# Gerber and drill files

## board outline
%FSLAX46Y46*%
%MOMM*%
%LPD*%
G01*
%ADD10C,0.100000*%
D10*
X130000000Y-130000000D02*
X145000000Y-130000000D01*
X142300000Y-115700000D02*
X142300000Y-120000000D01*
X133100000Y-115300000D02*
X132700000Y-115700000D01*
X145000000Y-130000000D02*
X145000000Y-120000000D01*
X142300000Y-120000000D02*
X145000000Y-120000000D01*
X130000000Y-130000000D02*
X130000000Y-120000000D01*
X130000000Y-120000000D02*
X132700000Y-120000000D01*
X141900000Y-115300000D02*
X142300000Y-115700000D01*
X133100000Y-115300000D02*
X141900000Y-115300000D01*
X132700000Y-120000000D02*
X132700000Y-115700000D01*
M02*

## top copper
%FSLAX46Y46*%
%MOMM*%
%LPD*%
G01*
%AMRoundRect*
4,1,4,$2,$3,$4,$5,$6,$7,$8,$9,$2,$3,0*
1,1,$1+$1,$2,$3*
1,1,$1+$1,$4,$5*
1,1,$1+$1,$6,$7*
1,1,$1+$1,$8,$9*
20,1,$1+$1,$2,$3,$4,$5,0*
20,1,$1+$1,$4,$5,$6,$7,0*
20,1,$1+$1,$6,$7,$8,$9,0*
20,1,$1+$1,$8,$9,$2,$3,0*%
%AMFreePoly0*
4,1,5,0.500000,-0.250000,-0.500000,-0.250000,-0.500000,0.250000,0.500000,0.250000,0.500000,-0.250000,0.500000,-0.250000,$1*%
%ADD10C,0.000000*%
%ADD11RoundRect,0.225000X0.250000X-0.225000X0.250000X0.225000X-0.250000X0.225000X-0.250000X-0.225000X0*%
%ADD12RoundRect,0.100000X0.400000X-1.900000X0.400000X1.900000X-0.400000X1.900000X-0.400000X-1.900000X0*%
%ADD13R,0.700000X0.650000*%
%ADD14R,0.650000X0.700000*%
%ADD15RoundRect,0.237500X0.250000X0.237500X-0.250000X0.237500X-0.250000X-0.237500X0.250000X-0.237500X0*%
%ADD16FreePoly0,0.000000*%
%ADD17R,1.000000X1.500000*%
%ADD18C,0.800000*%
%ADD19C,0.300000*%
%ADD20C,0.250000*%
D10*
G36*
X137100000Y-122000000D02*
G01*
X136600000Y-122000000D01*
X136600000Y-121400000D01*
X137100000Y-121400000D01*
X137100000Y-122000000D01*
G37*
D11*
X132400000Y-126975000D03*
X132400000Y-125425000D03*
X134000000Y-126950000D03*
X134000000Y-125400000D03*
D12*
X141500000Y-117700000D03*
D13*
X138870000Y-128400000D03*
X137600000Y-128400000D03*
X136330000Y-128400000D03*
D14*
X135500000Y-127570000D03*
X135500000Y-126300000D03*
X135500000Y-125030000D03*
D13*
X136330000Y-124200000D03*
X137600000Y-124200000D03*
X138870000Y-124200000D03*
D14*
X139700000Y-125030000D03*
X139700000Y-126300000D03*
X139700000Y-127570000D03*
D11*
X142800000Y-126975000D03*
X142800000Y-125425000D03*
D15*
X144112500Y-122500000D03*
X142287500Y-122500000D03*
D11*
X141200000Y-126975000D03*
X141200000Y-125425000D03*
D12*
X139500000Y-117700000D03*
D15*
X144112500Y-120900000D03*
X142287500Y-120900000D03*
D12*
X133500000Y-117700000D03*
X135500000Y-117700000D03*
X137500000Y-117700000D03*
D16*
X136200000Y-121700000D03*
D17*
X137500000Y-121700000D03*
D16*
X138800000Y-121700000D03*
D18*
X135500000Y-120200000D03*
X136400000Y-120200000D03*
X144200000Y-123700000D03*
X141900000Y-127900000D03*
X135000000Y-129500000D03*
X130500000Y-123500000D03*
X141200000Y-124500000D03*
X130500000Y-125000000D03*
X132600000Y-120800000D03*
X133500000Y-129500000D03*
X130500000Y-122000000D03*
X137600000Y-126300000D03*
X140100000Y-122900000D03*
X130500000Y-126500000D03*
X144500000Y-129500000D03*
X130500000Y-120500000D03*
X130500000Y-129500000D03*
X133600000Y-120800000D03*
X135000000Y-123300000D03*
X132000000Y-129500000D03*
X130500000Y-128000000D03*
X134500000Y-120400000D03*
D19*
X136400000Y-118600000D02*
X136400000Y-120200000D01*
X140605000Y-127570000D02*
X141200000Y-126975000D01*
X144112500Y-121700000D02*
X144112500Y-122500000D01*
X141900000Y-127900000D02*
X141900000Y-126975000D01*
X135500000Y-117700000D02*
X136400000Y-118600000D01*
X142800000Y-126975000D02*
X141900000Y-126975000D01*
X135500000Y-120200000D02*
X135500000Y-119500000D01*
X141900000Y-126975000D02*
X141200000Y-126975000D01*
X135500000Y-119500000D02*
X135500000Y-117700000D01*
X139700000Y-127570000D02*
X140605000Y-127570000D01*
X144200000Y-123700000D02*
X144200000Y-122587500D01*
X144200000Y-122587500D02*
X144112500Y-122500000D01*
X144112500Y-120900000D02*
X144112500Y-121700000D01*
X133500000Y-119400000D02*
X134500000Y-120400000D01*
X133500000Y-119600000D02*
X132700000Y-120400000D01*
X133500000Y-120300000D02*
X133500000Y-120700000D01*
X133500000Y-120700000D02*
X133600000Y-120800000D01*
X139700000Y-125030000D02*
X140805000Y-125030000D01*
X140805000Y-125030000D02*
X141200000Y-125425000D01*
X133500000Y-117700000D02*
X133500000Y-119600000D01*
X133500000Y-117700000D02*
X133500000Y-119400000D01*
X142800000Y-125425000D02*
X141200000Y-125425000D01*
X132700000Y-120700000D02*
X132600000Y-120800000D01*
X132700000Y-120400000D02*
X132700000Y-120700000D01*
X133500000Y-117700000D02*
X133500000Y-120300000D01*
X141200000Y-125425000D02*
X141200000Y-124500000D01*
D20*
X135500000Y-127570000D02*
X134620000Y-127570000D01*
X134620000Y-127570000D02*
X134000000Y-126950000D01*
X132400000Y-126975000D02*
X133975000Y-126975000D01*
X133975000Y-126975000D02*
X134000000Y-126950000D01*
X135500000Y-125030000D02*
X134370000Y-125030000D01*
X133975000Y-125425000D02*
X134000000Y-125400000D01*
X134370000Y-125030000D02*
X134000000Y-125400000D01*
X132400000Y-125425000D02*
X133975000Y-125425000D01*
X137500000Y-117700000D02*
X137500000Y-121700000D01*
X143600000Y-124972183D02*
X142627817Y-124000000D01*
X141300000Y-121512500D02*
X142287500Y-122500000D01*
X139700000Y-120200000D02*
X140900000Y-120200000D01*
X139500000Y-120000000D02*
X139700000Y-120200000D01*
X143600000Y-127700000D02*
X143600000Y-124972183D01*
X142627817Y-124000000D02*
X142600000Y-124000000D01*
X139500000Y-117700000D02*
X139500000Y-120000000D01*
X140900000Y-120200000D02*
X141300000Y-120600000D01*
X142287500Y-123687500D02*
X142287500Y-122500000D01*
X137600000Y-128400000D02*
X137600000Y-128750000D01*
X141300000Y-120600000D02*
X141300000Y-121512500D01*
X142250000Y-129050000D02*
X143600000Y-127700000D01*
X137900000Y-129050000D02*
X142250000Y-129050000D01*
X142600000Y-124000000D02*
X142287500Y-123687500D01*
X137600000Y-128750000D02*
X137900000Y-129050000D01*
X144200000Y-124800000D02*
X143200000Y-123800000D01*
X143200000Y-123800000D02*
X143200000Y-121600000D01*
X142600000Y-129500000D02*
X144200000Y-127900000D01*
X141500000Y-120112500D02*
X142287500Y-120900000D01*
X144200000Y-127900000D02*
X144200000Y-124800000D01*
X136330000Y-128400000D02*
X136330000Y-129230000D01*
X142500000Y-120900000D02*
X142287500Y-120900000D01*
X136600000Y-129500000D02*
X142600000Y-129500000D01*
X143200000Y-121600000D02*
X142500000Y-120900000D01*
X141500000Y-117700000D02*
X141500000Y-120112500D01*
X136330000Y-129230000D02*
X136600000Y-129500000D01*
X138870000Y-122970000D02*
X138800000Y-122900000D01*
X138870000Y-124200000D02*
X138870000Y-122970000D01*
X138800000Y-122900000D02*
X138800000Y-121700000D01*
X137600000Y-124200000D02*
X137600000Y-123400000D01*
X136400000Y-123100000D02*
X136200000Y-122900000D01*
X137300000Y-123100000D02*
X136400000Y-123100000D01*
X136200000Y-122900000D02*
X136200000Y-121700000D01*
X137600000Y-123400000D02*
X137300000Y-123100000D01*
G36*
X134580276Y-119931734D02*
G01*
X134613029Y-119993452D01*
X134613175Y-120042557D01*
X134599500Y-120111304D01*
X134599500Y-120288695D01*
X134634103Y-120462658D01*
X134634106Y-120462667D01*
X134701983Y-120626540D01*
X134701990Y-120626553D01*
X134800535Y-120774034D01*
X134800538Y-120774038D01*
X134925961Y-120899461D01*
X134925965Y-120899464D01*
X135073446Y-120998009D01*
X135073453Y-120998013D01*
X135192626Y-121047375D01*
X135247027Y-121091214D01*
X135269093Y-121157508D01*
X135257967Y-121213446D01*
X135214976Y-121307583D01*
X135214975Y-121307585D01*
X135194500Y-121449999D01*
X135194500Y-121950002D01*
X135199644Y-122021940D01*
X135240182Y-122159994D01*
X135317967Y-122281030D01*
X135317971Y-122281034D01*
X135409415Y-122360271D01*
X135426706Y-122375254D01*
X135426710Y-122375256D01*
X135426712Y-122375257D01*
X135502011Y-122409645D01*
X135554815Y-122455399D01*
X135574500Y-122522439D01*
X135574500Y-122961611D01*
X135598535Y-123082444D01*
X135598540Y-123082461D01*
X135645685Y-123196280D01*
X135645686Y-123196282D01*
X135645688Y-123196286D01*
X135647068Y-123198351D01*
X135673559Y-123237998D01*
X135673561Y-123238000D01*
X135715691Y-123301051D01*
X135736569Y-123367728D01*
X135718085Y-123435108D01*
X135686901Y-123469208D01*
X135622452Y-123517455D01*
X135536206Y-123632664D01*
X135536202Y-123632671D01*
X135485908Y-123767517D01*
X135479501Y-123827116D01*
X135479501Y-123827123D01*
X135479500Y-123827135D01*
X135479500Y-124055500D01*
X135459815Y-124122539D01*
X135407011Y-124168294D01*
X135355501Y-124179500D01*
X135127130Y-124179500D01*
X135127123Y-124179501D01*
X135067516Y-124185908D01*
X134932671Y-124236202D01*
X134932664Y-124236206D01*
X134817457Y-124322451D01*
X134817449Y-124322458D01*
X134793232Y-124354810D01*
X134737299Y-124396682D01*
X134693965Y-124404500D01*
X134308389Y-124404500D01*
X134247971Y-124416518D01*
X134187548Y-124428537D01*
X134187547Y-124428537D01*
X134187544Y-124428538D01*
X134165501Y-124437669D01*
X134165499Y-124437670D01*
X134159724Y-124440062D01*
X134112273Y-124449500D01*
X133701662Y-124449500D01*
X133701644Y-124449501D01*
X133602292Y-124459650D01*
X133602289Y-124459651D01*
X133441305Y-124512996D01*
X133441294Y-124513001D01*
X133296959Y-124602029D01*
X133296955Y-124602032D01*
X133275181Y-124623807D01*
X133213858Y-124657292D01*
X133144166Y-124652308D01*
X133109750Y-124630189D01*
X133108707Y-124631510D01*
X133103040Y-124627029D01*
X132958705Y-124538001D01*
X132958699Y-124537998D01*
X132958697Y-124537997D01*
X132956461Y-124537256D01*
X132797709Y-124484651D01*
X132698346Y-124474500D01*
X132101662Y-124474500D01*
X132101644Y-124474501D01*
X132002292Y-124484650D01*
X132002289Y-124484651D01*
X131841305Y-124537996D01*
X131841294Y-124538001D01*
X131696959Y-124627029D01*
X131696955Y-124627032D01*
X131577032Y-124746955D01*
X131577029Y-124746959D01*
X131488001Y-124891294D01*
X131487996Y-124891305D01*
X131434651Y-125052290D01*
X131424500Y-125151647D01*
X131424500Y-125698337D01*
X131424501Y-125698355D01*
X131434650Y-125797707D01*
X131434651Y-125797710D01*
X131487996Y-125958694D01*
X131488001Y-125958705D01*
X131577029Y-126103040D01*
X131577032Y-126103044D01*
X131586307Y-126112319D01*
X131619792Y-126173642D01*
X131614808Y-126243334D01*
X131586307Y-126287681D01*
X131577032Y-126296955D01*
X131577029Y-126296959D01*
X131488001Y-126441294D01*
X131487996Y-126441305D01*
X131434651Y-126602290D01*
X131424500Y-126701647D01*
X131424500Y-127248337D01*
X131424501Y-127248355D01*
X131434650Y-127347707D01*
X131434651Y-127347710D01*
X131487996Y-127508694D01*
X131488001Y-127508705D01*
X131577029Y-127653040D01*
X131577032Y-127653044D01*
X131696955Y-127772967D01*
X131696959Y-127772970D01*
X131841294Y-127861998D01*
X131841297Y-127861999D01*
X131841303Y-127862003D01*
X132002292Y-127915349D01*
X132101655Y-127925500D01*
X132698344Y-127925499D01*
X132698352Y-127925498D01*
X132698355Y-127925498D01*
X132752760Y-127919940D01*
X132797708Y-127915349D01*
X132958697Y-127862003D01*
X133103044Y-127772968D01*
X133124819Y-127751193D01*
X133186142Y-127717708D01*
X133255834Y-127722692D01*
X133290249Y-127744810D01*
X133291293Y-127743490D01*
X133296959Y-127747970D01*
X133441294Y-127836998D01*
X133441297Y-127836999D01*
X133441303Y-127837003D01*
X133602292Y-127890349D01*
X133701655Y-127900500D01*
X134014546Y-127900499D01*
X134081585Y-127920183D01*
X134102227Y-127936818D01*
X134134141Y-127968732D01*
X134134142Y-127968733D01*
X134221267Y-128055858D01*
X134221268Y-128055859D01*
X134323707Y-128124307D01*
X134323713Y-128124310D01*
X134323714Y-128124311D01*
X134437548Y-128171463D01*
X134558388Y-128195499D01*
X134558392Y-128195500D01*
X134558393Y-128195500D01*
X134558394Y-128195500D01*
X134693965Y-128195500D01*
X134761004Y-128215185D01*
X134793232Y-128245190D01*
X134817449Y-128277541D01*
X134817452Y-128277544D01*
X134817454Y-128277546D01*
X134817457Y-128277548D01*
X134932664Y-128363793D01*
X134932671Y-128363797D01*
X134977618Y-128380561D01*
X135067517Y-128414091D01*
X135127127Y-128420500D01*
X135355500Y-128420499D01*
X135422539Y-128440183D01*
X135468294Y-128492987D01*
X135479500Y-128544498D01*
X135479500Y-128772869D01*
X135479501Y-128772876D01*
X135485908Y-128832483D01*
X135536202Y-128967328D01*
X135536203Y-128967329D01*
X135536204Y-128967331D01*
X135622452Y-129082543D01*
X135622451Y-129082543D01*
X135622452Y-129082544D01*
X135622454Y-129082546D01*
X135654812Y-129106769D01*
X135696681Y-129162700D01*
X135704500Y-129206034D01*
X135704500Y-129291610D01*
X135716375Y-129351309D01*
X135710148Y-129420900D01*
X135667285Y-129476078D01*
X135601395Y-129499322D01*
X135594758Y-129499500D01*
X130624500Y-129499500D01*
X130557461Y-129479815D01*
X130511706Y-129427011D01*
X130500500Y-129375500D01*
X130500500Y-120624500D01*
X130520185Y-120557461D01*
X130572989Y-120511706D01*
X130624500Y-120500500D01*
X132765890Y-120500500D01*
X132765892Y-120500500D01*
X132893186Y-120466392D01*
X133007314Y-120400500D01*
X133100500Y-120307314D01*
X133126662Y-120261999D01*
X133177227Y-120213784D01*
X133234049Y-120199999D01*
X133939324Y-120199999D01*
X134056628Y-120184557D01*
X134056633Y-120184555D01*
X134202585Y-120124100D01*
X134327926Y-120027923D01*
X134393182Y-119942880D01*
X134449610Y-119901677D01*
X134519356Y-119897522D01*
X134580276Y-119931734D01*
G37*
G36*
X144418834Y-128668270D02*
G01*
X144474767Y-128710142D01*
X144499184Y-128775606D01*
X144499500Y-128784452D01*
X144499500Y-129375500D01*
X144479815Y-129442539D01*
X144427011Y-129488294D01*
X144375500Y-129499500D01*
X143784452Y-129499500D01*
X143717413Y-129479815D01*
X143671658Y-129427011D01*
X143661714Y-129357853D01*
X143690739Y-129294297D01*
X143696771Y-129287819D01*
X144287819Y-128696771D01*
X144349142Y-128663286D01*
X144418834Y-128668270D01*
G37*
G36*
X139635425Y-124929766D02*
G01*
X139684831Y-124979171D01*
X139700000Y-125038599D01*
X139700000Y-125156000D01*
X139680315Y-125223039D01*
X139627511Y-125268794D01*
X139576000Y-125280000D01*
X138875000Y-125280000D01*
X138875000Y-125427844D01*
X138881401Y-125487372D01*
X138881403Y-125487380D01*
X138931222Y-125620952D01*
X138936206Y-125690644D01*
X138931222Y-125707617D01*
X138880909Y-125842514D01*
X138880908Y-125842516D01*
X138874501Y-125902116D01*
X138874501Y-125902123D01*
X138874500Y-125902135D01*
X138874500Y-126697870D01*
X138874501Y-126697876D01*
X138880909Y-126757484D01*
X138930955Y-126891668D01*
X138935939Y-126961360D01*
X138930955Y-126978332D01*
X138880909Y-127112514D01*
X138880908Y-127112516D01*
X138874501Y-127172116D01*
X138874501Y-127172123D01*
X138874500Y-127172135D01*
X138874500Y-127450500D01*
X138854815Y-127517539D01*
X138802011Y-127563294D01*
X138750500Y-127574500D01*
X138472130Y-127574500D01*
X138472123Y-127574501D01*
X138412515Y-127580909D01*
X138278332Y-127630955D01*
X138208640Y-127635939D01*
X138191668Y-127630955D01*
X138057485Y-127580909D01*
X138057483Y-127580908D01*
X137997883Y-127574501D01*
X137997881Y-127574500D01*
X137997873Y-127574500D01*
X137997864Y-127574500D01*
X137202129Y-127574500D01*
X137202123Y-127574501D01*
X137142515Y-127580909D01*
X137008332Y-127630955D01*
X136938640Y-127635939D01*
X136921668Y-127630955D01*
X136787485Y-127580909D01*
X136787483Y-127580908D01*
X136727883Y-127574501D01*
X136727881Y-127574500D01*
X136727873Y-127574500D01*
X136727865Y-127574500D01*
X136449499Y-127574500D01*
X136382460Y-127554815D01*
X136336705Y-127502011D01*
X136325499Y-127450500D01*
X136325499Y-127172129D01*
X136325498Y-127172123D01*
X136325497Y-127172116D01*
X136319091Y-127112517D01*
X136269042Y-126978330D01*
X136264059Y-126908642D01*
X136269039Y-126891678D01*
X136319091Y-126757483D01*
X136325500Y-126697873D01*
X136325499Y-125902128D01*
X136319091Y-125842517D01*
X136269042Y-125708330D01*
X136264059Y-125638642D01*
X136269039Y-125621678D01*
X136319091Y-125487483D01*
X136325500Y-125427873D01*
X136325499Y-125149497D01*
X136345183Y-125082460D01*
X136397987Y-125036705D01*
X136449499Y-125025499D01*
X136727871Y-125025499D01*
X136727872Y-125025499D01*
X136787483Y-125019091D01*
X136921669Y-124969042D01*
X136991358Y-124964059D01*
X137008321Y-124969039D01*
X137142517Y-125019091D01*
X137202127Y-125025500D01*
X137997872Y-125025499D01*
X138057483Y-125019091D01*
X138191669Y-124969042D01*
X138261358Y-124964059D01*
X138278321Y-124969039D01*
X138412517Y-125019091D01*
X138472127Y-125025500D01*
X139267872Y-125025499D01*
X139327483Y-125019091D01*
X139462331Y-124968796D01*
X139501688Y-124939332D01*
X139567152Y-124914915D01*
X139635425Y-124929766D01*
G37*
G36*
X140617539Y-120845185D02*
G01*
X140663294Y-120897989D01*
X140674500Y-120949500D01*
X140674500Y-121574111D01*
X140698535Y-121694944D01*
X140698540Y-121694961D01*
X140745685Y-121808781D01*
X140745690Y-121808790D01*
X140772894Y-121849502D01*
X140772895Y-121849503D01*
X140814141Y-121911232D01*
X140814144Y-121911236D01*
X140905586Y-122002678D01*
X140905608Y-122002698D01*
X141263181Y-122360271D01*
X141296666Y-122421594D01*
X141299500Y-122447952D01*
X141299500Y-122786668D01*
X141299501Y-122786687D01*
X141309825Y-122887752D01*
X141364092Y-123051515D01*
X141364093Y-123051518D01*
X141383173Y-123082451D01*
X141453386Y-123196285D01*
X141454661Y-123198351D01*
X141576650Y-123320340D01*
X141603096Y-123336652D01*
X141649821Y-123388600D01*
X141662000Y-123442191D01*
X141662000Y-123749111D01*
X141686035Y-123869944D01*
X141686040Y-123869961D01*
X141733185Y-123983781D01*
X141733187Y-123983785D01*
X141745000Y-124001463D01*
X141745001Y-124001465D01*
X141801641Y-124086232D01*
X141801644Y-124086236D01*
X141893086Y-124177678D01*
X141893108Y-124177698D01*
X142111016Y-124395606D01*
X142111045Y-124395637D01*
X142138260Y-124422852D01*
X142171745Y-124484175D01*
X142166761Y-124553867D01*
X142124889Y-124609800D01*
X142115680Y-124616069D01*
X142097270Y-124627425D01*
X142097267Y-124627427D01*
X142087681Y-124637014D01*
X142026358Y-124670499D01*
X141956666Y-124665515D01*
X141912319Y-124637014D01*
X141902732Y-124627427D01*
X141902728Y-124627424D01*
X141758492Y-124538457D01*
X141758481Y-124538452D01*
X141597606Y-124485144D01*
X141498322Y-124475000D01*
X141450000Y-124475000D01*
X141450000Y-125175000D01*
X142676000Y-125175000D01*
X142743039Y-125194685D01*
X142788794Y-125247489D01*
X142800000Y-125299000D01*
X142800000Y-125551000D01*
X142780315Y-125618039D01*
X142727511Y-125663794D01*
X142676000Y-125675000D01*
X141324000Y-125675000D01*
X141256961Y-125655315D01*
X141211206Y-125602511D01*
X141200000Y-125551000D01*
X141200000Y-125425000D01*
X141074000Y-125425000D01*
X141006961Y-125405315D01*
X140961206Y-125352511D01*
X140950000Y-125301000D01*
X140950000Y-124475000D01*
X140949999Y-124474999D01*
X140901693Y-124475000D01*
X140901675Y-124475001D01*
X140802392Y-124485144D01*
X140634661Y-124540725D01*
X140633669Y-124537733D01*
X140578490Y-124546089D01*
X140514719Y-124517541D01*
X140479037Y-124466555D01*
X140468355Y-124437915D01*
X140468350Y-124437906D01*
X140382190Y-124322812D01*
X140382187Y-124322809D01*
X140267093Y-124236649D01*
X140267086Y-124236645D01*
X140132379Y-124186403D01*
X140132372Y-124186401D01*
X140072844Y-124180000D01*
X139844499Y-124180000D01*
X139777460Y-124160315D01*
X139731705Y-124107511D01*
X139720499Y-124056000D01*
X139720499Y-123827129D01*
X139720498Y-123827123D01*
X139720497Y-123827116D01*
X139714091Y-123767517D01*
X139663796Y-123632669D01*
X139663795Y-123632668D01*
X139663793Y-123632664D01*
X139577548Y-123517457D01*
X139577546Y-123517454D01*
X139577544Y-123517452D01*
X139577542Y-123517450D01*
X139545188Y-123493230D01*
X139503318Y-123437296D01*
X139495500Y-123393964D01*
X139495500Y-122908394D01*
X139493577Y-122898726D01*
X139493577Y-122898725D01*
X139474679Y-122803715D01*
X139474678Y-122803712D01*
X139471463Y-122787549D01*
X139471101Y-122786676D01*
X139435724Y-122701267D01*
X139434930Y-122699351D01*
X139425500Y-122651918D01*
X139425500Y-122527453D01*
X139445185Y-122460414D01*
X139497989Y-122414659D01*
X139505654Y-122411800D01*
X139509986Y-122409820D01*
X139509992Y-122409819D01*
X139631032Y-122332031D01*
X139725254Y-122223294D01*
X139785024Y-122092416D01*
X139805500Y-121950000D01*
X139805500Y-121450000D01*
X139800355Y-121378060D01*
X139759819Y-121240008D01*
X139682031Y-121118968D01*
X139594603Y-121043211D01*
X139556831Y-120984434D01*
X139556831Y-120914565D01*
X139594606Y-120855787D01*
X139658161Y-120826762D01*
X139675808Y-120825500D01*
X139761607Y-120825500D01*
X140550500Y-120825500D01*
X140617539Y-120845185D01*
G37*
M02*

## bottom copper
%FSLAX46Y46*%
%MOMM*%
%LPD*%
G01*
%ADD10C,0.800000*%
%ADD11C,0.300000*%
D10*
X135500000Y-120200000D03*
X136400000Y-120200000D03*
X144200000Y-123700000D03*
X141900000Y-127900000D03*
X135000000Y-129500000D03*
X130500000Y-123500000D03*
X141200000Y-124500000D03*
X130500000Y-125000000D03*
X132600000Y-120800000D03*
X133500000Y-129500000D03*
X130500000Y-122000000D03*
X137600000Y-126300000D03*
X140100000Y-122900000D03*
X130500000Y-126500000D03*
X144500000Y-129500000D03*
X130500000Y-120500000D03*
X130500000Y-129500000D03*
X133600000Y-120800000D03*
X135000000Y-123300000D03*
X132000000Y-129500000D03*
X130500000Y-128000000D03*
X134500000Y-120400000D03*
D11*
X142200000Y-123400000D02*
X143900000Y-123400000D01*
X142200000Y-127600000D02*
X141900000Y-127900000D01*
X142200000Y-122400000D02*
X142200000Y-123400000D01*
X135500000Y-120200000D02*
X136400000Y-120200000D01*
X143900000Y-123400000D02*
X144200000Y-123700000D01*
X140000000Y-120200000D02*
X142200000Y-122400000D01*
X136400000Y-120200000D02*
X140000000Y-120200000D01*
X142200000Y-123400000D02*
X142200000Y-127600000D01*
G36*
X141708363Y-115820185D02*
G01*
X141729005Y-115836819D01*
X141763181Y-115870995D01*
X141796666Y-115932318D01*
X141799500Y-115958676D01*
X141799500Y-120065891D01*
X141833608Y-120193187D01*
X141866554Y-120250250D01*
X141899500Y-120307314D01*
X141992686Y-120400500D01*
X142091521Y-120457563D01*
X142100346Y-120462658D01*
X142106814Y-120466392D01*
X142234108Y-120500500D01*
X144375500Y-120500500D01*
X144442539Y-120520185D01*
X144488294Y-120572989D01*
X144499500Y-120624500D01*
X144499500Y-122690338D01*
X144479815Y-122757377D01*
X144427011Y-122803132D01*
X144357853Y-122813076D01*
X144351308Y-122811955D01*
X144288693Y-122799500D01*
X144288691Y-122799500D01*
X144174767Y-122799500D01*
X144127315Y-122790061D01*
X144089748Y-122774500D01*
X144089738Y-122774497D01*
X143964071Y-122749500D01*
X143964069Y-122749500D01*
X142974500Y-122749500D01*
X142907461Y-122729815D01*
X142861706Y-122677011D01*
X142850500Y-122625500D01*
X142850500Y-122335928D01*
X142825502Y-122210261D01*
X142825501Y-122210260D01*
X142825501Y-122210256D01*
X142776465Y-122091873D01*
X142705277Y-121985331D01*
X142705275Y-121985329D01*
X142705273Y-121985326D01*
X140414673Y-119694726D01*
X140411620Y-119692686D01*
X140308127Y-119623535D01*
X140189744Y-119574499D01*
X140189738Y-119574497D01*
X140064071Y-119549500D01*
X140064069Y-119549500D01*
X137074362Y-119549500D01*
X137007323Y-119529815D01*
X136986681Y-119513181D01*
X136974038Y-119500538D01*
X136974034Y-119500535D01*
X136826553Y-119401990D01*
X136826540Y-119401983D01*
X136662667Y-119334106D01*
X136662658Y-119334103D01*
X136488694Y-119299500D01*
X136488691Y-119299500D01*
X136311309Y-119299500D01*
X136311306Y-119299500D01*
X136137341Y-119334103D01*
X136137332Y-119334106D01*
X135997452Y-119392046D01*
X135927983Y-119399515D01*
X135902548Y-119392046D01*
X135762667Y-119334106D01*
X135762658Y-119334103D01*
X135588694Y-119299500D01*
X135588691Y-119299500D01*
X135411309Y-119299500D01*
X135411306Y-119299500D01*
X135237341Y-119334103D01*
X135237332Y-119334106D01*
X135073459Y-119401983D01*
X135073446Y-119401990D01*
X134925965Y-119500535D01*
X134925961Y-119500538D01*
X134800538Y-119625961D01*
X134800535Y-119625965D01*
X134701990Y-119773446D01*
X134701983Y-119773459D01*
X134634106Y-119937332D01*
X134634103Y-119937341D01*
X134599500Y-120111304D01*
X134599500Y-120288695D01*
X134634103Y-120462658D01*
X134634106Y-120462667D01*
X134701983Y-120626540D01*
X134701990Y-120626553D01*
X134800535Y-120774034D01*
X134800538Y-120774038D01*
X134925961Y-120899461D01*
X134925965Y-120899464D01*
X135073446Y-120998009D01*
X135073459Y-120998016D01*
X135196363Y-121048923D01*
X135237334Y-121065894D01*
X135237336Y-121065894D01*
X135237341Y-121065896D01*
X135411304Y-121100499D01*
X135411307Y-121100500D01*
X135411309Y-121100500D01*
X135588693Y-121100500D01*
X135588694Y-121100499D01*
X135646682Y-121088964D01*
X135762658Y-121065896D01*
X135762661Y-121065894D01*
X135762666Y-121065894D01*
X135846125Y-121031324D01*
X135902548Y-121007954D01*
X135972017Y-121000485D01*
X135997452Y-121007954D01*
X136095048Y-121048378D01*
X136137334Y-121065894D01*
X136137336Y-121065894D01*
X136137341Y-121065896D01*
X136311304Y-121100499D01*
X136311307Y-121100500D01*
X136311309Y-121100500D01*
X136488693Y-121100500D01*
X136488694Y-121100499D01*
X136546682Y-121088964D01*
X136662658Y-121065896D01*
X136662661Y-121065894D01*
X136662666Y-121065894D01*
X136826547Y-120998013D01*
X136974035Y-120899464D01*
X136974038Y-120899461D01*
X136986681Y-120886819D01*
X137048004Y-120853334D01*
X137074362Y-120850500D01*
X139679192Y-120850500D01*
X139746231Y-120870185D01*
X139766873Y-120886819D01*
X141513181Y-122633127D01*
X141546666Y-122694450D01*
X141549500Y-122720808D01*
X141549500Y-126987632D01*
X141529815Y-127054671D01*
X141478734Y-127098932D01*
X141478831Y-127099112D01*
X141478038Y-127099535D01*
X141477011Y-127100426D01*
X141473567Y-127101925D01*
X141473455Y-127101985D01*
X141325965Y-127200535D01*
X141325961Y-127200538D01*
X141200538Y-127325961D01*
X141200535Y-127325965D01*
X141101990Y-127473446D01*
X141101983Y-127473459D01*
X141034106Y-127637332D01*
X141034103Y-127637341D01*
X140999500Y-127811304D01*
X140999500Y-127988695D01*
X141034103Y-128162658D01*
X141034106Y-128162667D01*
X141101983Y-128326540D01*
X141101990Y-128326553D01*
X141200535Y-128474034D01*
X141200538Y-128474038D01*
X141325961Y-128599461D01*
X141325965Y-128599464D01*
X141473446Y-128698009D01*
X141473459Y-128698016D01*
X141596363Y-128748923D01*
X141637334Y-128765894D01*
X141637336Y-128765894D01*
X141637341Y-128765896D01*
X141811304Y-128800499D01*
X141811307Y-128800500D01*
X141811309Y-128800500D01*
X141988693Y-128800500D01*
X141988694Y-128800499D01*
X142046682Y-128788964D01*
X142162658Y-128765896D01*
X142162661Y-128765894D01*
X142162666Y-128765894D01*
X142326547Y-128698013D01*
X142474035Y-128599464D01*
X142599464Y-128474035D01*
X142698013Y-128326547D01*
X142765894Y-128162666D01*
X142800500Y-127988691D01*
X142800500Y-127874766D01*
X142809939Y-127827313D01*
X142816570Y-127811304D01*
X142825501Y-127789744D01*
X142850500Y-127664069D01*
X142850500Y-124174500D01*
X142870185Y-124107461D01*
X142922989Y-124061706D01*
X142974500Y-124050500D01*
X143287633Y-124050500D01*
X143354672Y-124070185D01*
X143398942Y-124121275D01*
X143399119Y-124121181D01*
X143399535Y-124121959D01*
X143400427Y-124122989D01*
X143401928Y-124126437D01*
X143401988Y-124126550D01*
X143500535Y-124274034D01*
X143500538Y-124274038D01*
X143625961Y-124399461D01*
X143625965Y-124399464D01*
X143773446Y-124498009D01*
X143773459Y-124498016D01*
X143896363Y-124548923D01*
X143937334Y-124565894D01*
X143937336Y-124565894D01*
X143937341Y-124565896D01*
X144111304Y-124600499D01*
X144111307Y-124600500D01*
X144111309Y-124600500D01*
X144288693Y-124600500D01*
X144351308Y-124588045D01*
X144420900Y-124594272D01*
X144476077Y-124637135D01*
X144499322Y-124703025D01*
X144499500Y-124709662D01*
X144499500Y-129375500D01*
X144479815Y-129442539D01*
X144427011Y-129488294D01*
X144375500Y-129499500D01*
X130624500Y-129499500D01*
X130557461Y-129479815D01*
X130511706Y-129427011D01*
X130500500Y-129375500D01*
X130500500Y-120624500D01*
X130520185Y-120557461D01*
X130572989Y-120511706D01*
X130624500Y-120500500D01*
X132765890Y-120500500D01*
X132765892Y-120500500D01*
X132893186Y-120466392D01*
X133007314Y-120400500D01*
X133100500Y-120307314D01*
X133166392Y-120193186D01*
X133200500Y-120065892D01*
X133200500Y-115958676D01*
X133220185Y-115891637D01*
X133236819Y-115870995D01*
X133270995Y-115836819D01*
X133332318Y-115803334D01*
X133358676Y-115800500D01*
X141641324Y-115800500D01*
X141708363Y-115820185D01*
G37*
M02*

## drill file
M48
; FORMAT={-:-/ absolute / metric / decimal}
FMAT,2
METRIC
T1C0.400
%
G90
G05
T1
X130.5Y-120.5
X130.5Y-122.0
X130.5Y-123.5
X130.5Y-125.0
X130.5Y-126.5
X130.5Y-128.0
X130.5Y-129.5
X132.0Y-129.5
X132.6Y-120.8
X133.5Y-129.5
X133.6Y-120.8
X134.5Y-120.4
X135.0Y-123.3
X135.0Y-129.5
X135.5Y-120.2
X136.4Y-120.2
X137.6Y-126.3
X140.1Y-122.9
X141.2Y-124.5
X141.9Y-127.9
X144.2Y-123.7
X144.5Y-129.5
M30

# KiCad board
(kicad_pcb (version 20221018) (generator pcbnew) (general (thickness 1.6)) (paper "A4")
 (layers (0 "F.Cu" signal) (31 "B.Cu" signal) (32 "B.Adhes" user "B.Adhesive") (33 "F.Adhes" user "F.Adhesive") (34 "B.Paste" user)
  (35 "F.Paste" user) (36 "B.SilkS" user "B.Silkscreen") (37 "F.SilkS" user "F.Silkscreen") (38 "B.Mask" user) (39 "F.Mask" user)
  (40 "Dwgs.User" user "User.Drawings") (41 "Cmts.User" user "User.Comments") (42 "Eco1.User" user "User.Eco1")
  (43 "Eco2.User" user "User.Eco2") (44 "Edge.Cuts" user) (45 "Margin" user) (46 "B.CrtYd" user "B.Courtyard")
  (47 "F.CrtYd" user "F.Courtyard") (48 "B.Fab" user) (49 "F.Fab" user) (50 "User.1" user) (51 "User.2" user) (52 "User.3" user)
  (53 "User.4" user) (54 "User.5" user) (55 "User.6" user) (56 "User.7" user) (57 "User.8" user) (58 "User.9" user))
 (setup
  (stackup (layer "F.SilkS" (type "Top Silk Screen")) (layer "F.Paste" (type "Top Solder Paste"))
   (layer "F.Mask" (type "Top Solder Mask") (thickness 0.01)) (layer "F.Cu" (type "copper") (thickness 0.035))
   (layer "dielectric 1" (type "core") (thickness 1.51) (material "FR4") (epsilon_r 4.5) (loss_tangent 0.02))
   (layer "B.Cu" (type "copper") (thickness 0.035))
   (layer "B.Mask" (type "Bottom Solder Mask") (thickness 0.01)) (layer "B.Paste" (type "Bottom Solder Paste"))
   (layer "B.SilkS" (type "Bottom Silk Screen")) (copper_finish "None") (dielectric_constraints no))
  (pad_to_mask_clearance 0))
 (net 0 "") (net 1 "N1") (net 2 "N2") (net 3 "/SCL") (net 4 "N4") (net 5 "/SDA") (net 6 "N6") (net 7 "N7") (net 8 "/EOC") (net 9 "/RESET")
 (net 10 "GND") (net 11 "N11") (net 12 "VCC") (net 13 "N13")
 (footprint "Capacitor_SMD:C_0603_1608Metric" (layer "F.Cu") (at 132.4 126.2 90)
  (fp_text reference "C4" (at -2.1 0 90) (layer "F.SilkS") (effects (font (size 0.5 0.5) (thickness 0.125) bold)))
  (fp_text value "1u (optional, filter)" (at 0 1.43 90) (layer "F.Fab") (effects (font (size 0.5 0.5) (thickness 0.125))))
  (pad "1" smd roundrect (at -0.775 0 90) (size 0.9 0.95) (layers "F.Cu" "F.Paste" "F.Mask") (roundrect_rratio 0.25) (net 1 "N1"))
  (pad "2" smd roundrect (at 0.775 0 90) (size 0.9 0.95) (layers "F.Cu" "F.Paste" "F.Mask") (roundrect_rratio 0.25) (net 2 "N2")))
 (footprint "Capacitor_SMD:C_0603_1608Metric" (layer "F.Cu") (at 134 126.175 90)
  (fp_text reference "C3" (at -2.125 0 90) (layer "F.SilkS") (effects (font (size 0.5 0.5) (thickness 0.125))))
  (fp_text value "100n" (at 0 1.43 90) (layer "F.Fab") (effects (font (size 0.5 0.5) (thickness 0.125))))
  (pad "1" smd roundrect (at -0.775 0 90) (size 0.9 0.95) (layers "F.Cu" "F.Paste" "F.Mask") (roundrect_rratio 0.25) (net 1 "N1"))
  (pad "2" smd roundrect (at 0.775 0 90) (size 0.9 0.95) (layers "F.Cu" "F.Paste" "F.Mask") (roundrect_rratio 0.25) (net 2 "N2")))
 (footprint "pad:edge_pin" (layer "F.Cu") (at 141.5 117.7)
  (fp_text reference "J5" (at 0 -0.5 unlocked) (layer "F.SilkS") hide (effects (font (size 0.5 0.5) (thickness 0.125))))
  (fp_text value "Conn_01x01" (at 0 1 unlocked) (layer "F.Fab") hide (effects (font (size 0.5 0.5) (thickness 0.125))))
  (pad "1" smd roundrect (at 0 0 90) (size 4 1) (layers "F.Cu" "F.Mask") (roundrect_rratio 0.1) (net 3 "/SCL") (thermal_bridge_angle 45)))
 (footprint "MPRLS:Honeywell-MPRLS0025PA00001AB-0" (layer "F.Cu") (at 137.6 126.3)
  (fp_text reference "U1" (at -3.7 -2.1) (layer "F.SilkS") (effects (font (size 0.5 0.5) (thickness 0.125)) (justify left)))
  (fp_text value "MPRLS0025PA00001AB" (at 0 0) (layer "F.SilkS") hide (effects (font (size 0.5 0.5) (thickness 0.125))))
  (pad "1" smd rect (at 1.27 2.1) (size 0.7 0.65) (layers "F.Cu" "F.Paste" "F.Mask") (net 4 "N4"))
  (pad "2" smd rect (at 0 2.1) (size 0.7 0.65) (layers "F.Cu" "F.Paste" "F.Mask") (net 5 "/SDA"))
  (pad "3" smd rect (at -1.27 2.1) (size 0.7 0.65) (layers "F.Cu" "F.Paste" "F.Mask") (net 3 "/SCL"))
  (pad "4" smd rect (at -2.1 1.27) (size 0.65 0.7) (layers "F.Cu" "F.Paste" "F.Mask") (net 1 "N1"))
  (pad "5" smd rect (at -2.1 0) (size 0.65 0.7) (layers "F.Cu" "F.Paste" "F.Mask") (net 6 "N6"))
  (pad "6" smd rect (at -2.1 -1.27) (size 0.65 0.7) (layers "F.Cu" "F.Paste" "F.Mask") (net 2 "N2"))
  (pad "7" smd rect (at -1.27 -2.1) (size 0.7 0.65) (layers "F.Cu" "F.Paste" "F.Mask") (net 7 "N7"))
  (pad "8" smd rect (at 0 -2.1) (size 0.7 0.65) (layers "F.Cu" "F.Paste" "F.Mask") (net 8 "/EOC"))
  (pad "9" smd rect (at 1.27 -2.1) (size 0.7 0.65) (layers "F.Cu" "F.Paste" "F.Mask") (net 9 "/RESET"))
  (pad "10" smd rect (at 2.1 -1.27) (size 0.65 0.7) (layers "F.Cu" "F.Paste" "F.Mask") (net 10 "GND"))
  (pad "11" smd rect (at 2.1 0) (size 0.65 0.7) (layers "F.Cu" "F.Paste" "F.Mask") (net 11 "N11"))
  (pad "12" smd rect (at 2.1 1.27) (size 0.65 0.7) (layers "F.Cu" "F.Paste" "F.Mask") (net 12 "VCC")))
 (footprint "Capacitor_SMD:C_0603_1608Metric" (layer "F.Cu") (at 142.8 126.2 90)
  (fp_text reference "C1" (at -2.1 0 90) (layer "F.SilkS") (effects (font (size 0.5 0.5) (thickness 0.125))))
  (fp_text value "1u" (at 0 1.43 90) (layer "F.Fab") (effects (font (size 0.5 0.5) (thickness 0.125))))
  (pad "1" smd roundrect (at -0.775 0 90) (size 0.9 0.95) (layers "F.Cu" "F.Paste" "F.Mask") (roundrect_rratio 0.25) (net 12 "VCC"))
  (pad "2" smd roundrect (at 0.775 0 90) (size 0.9 0.95) (layers "F.Cu" "F.Paste" "F.Mask") (roundrect_rratio 0.25) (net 10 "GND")))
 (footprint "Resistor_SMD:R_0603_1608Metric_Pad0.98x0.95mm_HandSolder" (layer "F.Cu") (at 143.2 122.5 180)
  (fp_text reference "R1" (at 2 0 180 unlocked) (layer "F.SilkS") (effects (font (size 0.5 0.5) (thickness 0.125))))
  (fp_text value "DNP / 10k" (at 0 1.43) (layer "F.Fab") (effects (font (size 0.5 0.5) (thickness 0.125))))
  (pad "1" smd roundrect (at -0.9125 0 180) (size 0.975 0.95) (layers "F.Cu" "F.Paste" "F.Mask") (roundrect_rratio 0.25) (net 12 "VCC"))
  (pad "2" smd roundrect (at 0.9125 0 180) (size 0.975 0.95) (layers "F.Cu" "F.Paste" "F.Mask") (roundrect_rratio 0.25) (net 5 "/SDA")))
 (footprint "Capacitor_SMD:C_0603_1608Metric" (layer "F.Cu") (at 141.2 126.2 90)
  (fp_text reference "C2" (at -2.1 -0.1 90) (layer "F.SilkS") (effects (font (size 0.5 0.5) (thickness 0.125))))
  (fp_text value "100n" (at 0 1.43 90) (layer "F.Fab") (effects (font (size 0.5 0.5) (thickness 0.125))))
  (pad "1" smd roundrect (at -0.775 0 90) (size 0.9 0.95) (layers "F.Cu" "F.Paste" "F.Mask") (roundrect_rratio 0.25) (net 12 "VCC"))
  (pad "2" smd roundrect (at 0.775 0 90) (size 0.9 0.95) (layers "F.Cu" "F.Paste" "F.Mask") (roundrect_rratio 0.25) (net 10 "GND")))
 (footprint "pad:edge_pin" (layer "F.Cu") (at 139.5 117.7)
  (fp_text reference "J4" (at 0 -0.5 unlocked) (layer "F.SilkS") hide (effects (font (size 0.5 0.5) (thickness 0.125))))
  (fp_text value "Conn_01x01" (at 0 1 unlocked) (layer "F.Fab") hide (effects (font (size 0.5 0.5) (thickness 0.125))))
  (pad "1" smd roundrect (at 0 0 90) (size 4 1) (layers "F.Cu" "F.Mask") (roundrect_rratio 0.1) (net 5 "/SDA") (thermal_bridge_angle 45)))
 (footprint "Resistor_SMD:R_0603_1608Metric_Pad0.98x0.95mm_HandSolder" (layer "F.Cu") (at 143.2 120.9 180)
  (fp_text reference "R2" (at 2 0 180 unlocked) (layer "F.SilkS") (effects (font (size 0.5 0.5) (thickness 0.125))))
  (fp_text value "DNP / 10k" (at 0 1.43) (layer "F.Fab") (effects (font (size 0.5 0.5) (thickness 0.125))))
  (pad "1" smd roundrect (at -0.9125 0 180) (size 0.975 0.95) (layers "F.Cu" "F.Paste" "F.Mask") (roundrect_rratio 0.25) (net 12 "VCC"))
  (pad "2" smd roundrect (at 0.9125 0 180) (size 0.975 0.95) (layers "F.Cu" "F.Paste" "F.Mask") (roundrect_rratio 0.25) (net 3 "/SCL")))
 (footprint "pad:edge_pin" (layer "F.Cu") (at 133.5 117.7)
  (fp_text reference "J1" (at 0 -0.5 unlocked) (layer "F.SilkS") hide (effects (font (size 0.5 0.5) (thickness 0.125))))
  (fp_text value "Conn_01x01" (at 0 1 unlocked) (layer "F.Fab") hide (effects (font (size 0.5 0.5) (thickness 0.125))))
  (pad "1" smd roundrect (at 0 0 90) (size 4 1) (layers "F.Cu" "F.Mask") (roundrect_rratio 0.1) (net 10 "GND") (thermal_bridge_angle 45)))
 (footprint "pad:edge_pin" (layer "F.Cu") (at 135.5 117.7)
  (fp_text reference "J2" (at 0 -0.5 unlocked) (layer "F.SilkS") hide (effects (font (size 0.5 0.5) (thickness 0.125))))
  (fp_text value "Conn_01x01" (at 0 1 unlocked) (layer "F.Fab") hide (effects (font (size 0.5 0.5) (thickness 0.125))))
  (pad "1" smd roundrect (at 0 0 90) (size 4 1) (layers "F.Cu" "F.Mask") (roundrect_rratio 0.1) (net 12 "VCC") (thermal_bridge_angle 45)))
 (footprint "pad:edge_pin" (layer "F.Cu") (at 137.5 117.7)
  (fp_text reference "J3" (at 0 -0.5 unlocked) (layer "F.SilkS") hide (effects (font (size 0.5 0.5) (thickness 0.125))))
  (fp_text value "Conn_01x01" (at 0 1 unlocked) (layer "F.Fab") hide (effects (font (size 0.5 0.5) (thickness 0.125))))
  (pad "1" smd roundrect (at 0 0 90) (size 4 1) (layers "F.Cu" "F.Mask") (roundrect_rratio 0.1) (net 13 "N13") (thermal_bridge_angle 45)))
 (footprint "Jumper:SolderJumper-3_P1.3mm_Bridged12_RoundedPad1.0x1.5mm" (layer "F.Cu") (at 137.5 121.7) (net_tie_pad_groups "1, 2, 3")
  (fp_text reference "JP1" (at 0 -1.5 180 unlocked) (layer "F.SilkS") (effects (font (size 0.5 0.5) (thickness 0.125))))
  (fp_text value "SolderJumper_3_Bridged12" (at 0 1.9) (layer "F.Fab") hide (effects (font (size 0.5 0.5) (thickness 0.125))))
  (fp_poly (pts (xy -0.9 -0.3) (xy -0.4 -0.3) (xy -0.4 0.3) (xy -0.9 0.3)) (stroke (width 0) (type solid)) (fill solid) (layer "F.Cu"))
  (pad "1" smd custom (at -1.3 0) (size 1 0.5) (layers "F.Cu" "F.Mask") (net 8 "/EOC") (zone_connect 2) (thermal_bridge_angle 45)
   (options (clearance outline) (anchor rect)) (primitives))
  (pad "2" smd rect (at 0 0) (size 1 1.5) (layers "F.Cu" "F.Mask") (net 13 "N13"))
  (pad "3" smd custom (at 1.3 0) (size 1 0.5) (layers "F.Cu" "F.Mask") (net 9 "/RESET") (zone_connect 2) (thermal_bridge_angle 45)
   (options (clearance outline) (anchor rect)) (primitives)))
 (gr_line (start 130 130) (end 145 130) (stroke (width 0.1) (type default)) (layer "Edge.Cuts"))
 (gr_line (start 142.3 115.7) (end 142.3 120) (stroke (width 0.1) (type default)) (layer "Edge.Cuts"))
 (gr_line (start 133.1 115.3) (end 132.7 115.7) (stroke (width 0.1) (type default)) (layer "Edge.Cuts"))
 (gr_line (start 145 130) (end 145 120) (stroke (width 0.1) (type default)) (layer "Edge.Cuts"))
 (gr_line (start 142.3 120) (end 145 120) (stroke (width 0.1) (type default)) (layer "Edge.Cuts"))
 (gr_line (start 130 130) (end 130 120) (stroke (width 0.1) (type default)) (layer "Edge.Cuts"))
 (gr_line (start 130 120) (end 132.7 120) (stroke (width 0.1) (type default)) (layer "Edge.Cuts"))
 (gr_line (start 141.9 115.3) (end 142.3 115.7) (stroke (width 0.1) (type default)) (layer "Edge.Cuts"))
 (gr_line (start 133.1 115.3) (end 141.9 115.3) (stroke (width 0.1) (type default)) (layer "Edge.Cuts"))
 (gr_line (start 132.7 120) (end 132.7 115.7) (stroke (width 0.1) (type default)) (layer "Edge.Cuts"))
 (segment (start 136.4 118.6) (end 136.4 120.2) (width 0.3) (layer "F.Cu") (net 12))
 (segment (start 140.605 127.57) (end 141.2 126.975) (width 0.3) (layer "F.Cu") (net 12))
 (segment (start 144.1125 121.7) (end 144.1125 122.5) (width 0.3) (layer "F.Cu") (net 12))
 (segment (start 141.9 127.9) (end 141.9 126.975) (width 0.3) (layer "F.Cu") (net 12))
 (segment (start 135.5 117.7) (end 136.4 118.6) (width 0.3) (layer "F.Cu") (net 12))
 (segment (start 142.8 126.975) (end 141.9 126.975) (width 0.3) (layer "F.Cu") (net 12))
 (segment (start 135.5 120.2) (end 135.5 119.5) (width 0.3) (layer "F.Cu") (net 12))
 (segment (start 141.9 126.975) (end 141.2 126.975) (width 0.3) (layer "F.Cu") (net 12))
 (segment (start 135.5 119.5) (end 135.5 117.7) (width 0.3) (layer "F.Cu") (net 12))
 (segment (start 139.7 127.57) (end 140.605 127.57) (width 0.3) (layer "F.Cu") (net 12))
 (segment (start 144.2 123.7) (end 144.2 122.5875) (width 0.3) (layer "F.Cu") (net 12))
 (segment (start 144.2 122.5875) (end 144.1125 122.5) (width 0.3) (layer "F.Cu") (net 12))
 (segment (start 144.1125 120.9) (end 144.1125 121.7) (width 0.3) (layer "F.Cu") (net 12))
 (via (at 135.5 120.2) (size 0.8) (drill 0.4) (layers "F.Cu" "B.Cu") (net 12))
 (via (at 136.4 120.2) (size 0.8) (drill 0.4) (layers "F.Cu" "B.Cu") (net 12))
 (via (at 144.2 123.7) (size 0.8) (drill 0.4) (layers "F.Cu" "B.Cu") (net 12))
 (via (at 141.9 127.9) (size 0.8) (drill 0.4) (layers "F.Cu" "B.Cu") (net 12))
 (segment (start 142.2 123.4) (end 143.9 123.4) (width 0.3) (layer "B.Cu") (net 12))
 (segment (start 142.2 127.6) (end 141.9 127.9) (width 0.3) (layer "B.Cu") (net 12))
 (segment (start 142.2 122.4) (end 142.2 123.4) (width 0.3) (layer "B.Cu") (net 12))
 (segment (start 135.5 120.2) (end 136.4 120.2) (width 0.3) (layer "B.Cu") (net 12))
 (segment (start 143.9 123.4) (end 144.2 123.7) (width 0.3) (layer "B.Cu") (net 12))
 (segment (start 140 120.2) (end 142.2 122.4) (width 0.3) (layer "B.Cu") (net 12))
 (segment (start 136.4 120.2) (end 140 120.2) (width 0.3) (layer "B.Cu") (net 12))
 (segment (start 142.2 123.4) (end 142.2 127.6) (width 0.3) (layer "B.Cu") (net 12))
 (segment (start 133.5 119.4) (end 134.5 120.4) (width 0.3) (layer "F.Cu") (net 10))
 (segment (start 133.5 119.6) (end 132.7 120.4) (width 0.3) (layer "F.Cu") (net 10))
 (segment (start 133.5 120.3) (end 133.5 120.7) (width 0.3) (layer "F.Cu") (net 10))
 (segment (start 133.5 120.7) (end 133.6 120.8) (width 0.3) (layer "F.Cu") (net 10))
 (segment (start 139.7 125.03) (end 140.805 125.03) (width 0.3) (layer "F.Cu") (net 10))
 (segment (start 140.805 125.03) (end 141.2 125.425) (width 0.3) (layer "F.Cu") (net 10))
 (segment (start 133.5 117.7) (end 133.5 119.6) (width 0.3) (layer "F.Cu") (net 10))
 (segment (start 133.5 117.7) (end 133.5 119.4) (width 0.3) (layer "F.Cu") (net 10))
 (segment (start 142.8 125.425) (end 141.2 125.425) (width 0.3) (layer "F.Cu") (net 10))
 (segment (start 132.7 120.7) (end 132.6 120.8) (width 0.3) (layer "F.Cu") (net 10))
 (segment (start 132.7 120.4) (end 132.7 120.7) (width 0.3) (layer "F.Cu") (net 10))
 (segment (start 133.5 117.7) (end 133.5 120.3) (width 0.3) (layer "F.Cu") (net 10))
 (segment (start 141.2 125.425) (end 141.2 124.5) (width 0.3) (layer "F.Cu") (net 10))
 (via (at 135 129.5) (size 0.8) (drill 0.4) (layers "F.Cu" "B.Cu") (free) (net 10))
 (via (at 130.5 123.5) (size 0.8) (drill 0.4) (layers "F.Cu" "B.Cu") (free) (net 10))
 (via (at 141.2 124.5) (size 0.8) (drill 0.4) (layers "F.Cu" "B.Cu") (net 10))
 (via (at 130.5 125) (size 0.8) (drill 0.4) (layers "F.Cu" "B.Cu") (free) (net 10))
 (via (at 132.6 120.8) (size 0.8) (drill 0.4) (layers "F.Cu" "B.Cu") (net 10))
 (via (at 133.5 129.5) (size 0.8) (drill 0.4) (layers "F.Cu" "B.Cu") (free) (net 10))
 (via (at 130.5 122) (size 0.8) (drill 0.4) (layers "F.Cu" "B.Cu") (free) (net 10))
 (via (at 137.6 126.3) (size 0.8) (drill 0.4) (layers "F.Cu" "B.Cu") (free) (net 10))
 (via (at 140.1 122.9) (size 0.8) (drill 0.4) (layers "F.Cu" "B.Cu") (free) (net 10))
 (via (at 130.5 126.5) (size 0.8) (drill 0.4) (layers "F.Cu" "B.Cu") (free) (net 10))
 (via (at 144.5 129.5) (size 0.8) (drill 0.4) (layers "F.Cu" "B.Cu") (free) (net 10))
 (via (at 130.5 120.5) (size 0.8) (drill 0.4) (layers "F.Cu" "B.Cu") (free) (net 10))
 (via (at 130.5 129.5) (size 0.8) (drill 0.4) (layers "F.Cu" "B.Cu") (free) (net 10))
 (via (at 133.6 120.8) (size 0.8) (drill 0.4) (layers "F.Cu" "B.Cu") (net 10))
 (via (at 135 123.3) (size 0.8) (drill 0.4) (layers "F.Cu" "B.Cu") (free) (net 10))
 (via (at 132 129.5) (size 0.8) (drill 0.4) (layers "F.Cu" "B.Cu") (free) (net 10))
 (via (at 130.5 128) (size 0.8) (drill 0.4) (layers "F.Cu" "B.Cu") (free) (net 10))
 (via (at 134.5 120.4) (size 0.8) (drill 0.4) (layers "F.Cu" "B.Cu") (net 10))
 (segment (start 135.5 127.57) (end 134.62 127.57) (width 0.25) (layer "F.Cu") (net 1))
 (segment (start 134.62 127.57) (end 134 126.95) (width 0.25) (layer "F.Cu") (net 1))
 (segment (start 132.4 126.975) (end 133.975 126.975) (width 0.25) (layer "F.Cu") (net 1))
 (segment (start 133.975 126.975) (end 134 126.95) (width 0.25) (layer "F.Cu") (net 1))
 (segment (start 135.5 125.03) (end 134.37 125.03) (width 0.25) (layer "F.Cu") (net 2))
 (segment (start 133.975 125.425) (end 134 125.4) (width 0.25) (layer "F.Cu") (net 2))
 (segment (start 134.37 125.03) (end 134 125.4) (width 0.25) (layer "F.Cu") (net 2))
 (segment (start 132.4 125.425) (end 133.975 125.425) (width 0.25) (layer "F.Cu") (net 2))
 (segment (start 137.5 117.7) (end 137.5 121.7) (width 0.25) (layer "F.Cu") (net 13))
 (segment (start 143.6 124.972183) (end 142.627817 124) (width 0.25) (layer "F.Cu") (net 5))
 (segment (start 141.3 121.5125) (end 142.2875 122.5) (width 0.25) (layer "F.Cu") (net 5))
 (segment (start 139.7 120.2) (end 140.9 120.2) (width 0.25) (layer "F.Cu") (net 5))
 (segment (start 139.5 120) (end 139.7 120.2) (width 0.25) (layer "F.Cu") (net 5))
 (segment (start 143.6 127.7) (end 143.6 124.972183) (width 0.25) (layer "F.Cu") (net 5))
 (segment (start 142.627817 124) (end 142.6 124) (width 0.25) (layer "F.Cu") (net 5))
 (segment (start 139.5 117.7) (end 139.5 120) (width 0.25) (layer "F.Cu") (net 5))
 (segment (start 140.9 120.2) (end 141.3 120.6) (width 0.25) (layer "F.Cu") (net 5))
 (segment (start 142.2875 123.6875) (end 142.2875 122.5) (width 0.25) (layer "F.Cu") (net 5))
 (segment (start 137.6 128.4) (end 137.6 128.75) (width 0.25) (layer "F.Cu") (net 5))
 (segment (start 141.3 120.6) (end 141.3 121.5125) (width 0.25) (layer "F.Cu") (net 5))
 (segment (start 142.25 129.05) (end 143.6 127.7) (width 0.25) (layer "F.Cu") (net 5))
 (segment (start 137.9 129.05) (end 142.25 129.05) (width 0.25) (layer "F.Cu") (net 5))
 (segment (start 142.6 124) (end 142.2875 123.6875) (width 0.25) (layer "F.Cu") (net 5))
 (segment (start 137.6 128.75) (end 137.9 129.05) (width 0.25) (layer "F.Cu") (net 5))
 (segment (start 144.2 124.8) (end 143.2 123.8) (width 0.25) (layer "F.Cu") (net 3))
 (segment (start 143.2 123.8) (end 143.2 121.6) (width 0.25) (layer "F.Cu") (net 3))
 (segment (start 142.6 129.5) (end 144.2 127.9) (width 0.25) (layer "F.Cu") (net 3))
 (segment (start 141.5 120.1125) (end 142.2875 120.9) (width 0.25) (layer "F.Cu") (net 3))
 (segment (start 144.2 127.9) (end 144.2 124.8) (width 0.25) (layer "F.Cu") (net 3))
 (segment (start 136.33 128.4) (end 136.33 129.23) (width 0.25) (layer "F.Cu") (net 3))
 (segment (start 142.5 120.9) (end 142.2875 120.9) (width 0.25) (layer "F.Cu") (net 3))
 (segment (start 136.6 129.5) (end 142.6 129.5) (width 0.25) (layer "F.Cu") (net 3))
 (segment (start 143.2 121.6) (end 142.5 120.9) (width 0.25) (layer "F.Cu") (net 3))
 (segment (start 141.5 117.7) (end 141.5 120.1125) (width 0.25) (layer "F.Cu") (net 3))
 (segment (start 136.33 129.23) (end 136.6 129.5) (width 0.25) (layer "F.Cu") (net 3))
 (segment (start 138.87 122.97) (end 138.8 122.9) (width 0.25) (layer "F.Cu") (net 9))
 (segment (start 138.87 124.2) (end 138.87 122.97) (width 0.25) (layer "F.Cu") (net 9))
 (segment (start 138.8 122.9) (end 138.8 121.7) (width 0.25) (layer "F.Cu") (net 9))
 (segment (start 137.6 124.2) (end 137.6 123.4) (width 0.25) (layer "F.Cu") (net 8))
 (segment (start 136.4 123.1) (end 136.2 122.9) (width 0.25) (layer "F.Cu") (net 8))
 (segment (start 137.3 123.1) (end 136.4 123.1) (width 0.25) (layer "F.Cu") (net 8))
 (segment (start 136.2 122.9) (end 136.2 121.7) (width 0.25) (layer "F.Cu") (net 8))
 (segment (start 137.6 123.4) (end 137.3 123.1) (width 0.25) (layer "F.Cu") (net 8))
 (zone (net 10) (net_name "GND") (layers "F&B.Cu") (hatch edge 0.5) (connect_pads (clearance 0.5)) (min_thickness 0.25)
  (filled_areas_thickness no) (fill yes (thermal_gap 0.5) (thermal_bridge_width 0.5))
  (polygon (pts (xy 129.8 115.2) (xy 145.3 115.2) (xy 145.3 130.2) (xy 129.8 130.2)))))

